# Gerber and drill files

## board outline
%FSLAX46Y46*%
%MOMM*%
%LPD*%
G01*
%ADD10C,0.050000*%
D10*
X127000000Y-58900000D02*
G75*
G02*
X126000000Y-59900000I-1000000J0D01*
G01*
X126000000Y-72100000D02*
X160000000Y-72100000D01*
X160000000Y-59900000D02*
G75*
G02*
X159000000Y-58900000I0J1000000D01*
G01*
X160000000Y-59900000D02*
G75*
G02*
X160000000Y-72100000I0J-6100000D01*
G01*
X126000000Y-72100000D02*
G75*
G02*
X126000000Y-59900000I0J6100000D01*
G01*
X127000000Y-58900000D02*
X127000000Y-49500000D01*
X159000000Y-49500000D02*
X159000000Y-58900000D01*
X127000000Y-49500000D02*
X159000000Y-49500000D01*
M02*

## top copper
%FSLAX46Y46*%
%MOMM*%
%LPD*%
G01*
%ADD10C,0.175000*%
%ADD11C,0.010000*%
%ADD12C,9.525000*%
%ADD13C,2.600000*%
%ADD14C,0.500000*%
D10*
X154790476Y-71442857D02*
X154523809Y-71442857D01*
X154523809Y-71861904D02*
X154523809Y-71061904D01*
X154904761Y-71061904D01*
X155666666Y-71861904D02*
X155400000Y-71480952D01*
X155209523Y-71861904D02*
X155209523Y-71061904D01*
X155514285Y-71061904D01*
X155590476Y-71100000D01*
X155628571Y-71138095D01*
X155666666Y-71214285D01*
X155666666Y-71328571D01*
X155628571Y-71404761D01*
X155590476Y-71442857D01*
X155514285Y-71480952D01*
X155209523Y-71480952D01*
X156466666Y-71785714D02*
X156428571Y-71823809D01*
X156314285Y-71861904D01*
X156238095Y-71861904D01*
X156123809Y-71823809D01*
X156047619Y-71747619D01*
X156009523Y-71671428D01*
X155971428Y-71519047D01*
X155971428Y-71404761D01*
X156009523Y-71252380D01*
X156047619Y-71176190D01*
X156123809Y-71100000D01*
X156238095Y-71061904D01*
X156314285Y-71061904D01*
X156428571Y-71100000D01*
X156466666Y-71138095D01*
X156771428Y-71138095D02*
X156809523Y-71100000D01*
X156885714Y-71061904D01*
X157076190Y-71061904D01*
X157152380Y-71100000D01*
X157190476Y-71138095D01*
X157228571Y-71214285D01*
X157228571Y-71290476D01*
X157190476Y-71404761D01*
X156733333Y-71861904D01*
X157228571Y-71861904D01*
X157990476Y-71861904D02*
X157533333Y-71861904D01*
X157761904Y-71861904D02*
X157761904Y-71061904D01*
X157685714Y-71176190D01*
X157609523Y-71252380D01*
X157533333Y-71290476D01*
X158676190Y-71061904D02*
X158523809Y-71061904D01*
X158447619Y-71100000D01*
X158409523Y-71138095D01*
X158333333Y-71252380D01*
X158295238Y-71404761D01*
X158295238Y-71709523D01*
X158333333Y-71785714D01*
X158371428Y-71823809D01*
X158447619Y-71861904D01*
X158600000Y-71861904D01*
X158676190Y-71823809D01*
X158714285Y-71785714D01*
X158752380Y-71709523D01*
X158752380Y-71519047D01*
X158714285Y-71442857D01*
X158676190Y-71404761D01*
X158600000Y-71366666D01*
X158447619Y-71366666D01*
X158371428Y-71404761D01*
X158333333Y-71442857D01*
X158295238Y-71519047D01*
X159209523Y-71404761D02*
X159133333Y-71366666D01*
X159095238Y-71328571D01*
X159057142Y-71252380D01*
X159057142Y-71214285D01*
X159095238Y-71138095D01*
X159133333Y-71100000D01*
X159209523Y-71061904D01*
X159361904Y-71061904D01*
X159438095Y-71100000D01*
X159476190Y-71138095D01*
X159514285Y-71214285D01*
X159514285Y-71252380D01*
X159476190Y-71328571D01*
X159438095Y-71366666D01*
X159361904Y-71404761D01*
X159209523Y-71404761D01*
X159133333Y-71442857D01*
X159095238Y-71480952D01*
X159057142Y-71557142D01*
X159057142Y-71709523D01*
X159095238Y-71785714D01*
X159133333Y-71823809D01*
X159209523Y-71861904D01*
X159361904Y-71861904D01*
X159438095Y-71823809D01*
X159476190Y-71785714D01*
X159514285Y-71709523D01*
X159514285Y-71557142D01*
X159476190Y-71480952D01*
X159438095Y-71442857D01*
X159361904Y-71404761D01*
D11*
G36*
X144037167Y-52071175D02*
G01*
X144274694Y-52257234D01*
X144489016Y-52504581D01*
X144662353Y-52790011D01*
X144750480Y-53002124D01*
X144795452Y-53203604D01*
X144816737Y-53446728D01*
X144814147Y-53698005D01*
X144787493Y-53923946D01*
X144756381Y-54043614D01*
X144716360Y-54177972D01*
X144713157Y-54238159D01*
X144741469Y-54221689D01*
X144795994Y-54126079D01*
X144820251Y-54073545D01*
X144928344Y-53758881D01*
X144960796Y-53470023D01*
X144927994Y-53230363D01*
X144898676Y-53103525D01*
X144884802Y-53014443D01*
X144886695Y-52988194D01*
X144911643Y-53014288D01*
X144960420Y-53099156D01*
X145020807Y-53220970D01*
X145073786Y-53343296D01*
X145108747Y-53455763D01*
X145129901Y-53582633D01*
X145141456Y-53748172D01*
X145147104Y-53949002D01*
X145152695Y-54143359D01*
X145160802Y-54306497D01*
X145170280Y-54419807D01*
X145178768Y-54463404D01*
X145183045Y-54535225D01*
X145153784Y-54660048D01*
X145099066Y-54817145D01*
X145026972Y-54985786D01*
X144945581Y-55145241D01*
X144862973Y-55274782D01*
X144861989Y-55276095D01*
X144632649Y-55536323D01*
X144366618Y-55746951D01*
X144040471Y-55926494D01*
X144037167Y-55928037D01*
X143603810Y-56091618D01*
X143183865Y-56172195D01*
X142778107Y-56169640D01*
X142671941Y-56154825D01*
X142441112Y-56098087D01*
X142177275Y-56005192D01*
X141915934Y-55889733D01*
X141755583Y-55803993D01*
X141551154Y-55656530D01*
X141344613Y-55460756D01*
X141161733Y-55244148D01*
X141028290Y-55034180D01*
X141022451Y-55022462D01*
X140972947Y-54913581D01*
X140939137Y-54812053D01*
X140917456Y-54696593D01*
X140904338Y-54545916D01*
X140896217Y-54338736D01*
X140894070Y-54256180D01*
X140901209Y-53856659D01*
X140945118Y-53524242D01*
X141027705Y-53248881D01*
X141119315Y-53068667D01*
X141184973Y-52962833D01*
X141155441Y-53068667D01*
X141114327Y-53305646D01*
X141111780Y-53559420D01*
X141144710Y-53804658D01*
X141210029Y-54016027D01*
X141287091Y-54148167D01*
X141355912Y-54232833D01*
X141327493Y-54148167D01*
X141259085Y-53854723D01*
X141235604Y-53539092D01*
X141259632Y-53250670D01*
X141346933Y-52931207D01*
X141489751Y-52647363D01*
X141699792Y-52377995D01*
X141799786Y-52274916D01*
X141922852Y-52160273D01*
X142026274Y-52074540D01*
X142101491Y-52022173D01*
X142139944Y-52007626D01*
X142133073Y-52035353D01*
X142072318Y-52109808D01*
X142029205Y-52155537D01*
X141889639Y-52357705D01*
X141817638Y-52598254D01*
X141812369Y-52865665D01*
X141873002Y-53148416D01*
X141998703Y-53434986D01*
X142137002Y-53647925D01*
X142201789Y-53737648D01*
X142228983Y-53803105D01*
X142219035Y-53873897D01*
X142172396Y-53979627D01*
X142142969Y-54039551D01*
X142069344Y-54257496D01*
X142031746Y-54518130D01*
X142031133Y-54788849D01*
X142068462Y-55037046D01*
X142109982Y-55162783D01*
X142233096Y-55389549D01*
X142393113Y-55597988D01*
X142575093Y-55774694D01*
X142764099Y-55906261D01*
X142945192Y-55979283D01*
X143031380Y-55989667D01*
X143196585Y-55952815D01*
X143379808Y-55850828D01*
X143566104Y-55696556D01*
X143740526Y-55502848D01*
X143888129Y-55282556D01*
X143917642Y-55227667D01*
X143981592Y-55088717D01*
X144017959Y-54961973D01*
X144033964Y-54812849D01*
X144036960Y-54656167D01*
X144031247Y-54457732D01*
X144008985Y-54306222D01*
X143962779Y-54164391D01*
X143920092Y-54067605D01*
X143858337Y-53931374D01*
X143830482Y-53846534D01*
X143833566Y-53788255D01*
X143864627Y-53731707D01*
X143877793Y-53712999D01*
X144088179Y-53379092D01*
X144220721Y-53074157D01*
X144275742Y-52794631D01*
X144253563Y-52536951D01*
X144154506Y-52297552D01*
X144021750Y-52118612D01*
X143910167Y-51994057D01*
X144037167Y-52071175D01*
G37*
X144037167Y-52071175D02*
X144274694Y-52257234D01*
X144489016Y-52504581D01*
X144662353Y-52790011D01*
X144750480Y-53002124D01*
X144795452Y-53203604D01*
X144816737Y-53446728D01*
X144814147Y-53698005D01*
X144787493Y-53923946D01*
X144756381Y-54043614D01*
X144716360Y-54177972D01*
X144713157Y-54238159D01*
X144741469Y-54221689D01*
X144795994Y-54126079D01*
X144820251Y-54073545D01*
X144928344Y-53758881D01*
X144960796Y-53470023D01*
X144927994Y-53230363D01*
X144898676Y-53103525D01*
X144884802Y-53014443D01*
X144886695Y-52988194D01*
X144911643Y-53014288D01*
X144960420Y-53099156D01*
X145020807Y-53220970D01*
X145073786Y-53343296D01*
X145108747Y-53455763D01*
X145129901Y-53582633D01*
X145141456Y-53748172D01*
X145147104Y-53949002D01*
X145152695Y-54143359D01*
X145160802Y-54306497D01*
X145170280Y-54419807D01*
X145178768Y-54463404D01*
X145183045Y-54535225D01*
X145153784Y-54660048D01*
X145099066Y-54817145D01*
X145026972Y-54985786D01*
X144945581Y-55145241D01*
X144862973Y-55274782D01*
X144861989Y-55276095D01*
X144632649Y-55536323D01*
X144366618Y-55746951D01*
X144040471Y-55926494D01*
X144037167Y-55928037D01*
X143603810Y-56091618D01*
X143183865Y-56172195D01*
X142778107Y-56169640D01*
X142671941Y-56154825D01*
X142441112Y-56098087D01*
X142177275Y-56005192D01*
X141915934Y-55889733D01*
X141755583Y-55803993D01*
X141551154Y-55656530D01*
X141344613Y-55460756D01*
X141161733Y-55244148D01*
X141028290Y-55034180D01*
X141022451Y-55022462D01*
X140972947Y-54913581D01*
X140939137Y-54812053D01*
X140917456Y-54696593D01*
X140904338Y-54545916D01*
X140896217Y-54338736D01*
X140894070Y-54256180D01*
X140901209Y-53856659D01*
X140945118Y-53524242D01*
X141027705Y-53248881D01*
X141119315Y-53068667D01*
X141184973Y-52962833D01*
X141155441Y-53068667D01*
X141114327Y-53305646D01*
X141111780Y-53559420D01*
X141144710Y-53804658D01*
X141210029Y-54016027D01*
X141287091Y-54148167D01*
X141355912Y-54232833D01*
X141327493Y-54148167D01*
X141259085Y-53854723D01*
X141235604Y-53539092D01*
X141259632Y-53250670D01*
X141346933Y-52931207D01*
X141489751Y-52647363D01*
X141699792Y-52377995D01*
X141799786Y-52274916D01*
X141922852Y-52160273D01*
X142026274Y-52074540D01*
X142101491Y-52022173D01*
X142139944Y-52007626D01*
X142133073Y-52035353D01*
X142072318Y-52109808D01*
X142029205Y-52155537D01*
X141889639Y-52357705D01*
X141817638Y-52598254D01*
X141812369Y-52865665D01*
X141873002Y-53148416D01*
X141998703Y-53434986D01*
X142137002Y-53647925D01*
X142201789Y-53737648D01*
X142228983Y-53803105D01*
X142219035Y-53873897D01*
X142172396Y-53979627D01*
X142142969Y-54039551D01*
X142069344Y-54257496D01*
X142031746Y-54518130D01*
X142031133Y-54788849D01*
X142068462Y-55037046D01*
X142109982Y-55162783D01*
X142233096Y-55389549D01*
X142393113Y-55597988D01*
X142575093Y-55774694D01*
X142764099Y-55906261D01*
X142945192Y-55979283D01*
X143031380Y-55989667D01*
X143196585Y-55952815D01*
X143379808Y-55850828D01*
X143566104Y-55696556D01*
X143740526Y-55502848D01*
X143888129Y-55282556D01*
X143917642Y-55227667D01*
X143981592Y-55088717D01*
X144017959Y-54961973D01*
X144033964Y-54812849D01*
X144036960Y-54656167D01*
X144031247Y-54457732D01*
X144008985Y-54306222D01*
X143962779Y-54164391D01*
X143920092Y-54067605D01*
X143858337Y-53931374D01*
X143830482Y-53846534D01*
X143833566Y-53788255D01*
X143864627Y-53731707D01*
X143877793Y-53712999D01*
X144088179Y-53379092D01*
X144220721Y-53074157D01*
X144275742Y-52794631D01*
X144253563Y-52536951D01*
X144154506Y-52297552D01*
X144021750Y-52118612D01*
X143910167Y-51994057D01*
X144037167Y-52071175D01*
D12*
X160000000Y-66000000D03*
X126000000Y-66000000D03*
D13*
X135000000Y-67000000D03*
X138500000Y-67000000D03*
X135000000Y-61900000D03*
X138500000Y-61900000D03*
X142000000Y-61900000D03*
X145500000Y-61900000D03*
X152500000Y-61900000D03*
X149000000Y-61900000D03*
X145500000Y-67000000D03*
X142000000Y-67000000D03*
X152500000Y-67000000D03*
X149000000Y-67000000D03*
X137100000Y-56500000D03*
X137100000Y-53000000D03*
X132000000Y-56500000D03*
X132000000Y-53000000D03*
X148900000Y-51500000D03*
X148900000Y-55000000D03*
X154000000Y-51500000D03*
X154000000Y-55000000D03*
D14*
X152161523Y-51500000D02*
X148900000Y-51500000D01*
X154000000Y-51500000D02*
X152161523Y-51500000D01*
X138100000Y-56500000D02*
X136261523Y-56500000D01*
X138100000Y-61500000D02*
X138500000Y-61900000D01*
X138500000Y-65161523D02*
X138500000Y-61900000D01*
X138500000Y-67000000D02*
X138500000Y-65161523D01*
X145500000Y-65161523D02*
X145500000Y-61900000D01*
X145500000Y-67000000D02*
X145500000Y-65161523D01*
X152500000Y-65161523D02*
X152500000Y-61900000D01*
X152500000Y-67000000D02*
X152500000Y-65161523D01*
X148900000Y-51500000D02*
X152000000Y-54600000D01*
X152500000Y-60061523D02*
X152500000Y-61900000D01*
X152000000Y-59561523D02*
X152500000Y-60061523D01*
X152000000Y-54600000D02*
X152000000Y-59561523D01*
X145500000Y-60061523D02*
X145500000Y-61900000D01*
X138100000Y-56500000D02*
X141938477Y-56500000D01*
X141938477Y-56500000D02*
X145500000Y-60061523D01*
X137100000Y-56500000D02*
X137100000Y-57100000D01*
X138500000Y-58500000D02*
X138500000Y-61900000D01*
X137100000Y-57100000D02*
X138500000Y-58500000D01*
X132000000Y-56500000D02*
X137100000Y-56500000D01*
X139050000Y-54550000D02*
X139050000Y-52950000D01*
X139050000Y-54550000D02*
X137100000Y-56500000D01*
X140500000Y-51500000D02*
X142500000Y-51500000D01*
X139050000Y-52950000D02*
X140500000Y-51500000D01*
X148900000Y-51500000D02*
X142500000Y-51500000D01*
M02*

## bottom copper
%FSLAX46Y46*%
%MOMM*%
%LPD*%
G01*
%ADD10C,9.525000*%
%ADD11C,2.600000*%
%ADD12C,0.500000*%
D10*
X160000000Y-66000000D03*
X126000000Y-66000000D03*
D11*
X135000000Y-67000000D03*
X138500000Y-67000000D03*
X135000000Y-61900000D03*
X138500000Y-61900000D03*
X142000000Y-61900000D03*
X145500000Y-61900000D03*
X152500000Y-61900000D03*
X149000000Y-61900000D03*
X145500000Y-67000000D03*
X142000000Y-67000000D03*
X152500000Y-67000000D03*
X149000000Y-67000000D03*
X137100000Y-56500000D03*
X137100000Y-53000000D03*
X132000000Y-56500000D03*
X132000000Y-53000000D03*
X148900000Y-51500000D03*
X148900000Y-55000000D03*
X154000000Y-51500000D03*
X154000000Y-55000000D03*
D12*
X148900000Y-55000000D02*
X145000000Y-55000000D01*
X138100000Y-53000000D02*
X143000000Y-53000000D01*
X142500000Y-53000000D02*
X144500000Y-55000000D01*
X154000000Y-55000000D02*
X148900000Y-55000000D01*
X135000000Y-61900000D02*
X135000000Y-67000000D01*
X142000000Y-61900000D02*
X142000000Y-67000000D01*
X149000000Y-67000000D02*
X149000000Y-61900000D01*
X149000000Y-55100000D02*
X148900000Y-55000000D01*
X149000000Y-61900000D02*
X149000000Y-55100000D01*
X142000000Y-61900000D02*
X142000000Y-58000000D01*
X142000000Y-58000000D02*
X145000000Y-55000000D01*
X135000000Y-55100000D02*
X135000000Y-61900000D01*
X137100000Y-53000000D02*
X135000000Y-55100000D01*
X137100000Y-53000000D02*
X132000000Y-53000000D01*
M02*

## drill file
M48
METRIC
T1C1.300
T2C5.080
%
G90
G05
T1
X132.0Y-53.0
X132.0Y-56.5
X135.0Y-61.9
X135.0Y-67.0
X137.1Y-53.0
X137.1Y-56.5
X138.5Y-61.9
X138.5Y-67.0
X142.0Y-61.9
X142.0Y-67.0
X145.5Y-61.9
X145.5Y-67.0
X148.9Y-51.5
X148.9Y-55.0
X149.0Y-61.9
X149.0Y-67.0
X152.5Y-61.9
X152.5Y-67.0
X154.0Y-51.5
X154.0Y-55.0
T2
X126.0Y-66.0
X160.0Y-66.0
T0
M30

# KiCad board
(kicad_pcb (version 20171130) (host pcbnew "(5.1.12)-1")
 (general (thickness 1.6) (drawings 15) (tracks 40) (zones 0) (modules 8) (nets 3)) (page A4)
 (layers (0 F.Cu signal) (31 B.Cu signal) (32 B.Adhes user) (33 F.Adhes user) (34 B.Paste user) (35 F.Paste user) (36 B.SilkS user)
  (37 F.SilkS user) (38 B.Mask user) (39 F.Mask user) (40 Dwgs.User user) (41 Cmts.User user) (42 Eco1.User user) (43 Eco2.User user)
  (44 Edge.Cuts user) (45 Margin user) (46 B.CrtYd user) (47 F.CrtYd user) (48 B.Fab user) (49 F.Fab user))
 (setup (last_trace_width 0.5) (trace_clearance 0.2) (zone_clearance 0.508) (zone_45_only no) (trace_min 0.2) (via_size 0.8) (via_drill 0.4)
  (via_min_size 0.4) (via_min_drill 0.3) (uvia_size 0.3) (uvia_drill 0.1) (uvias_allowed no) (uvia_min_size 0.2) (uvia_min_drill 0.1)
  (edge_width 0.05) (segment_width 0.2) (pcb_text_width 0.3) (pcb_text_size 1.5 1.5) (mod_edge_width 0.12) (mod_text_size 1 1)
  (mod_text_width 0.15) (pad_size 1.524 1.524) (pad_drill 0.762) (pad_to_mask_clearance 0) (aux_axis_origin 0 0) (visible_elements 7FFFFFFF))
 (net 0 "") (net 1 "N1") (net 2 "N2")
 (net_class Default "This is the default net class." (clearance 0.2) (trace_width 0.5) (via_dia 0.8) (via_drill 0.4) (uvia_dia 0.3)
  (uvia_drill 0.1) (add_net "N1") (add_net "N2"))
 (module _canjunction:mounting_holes (layer F.Cu) (at 126 66)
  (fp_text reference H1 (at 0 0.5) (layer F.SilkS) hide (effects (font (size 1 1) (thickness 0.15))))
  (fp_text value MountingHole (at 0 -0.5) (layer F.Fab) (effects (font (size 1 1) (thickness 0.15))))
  (pad "" thru_hole circle (at 34 0) (size 9.525 9.525) (drill 5.08) (layers *.Cu *.Mask))
  (pad "" thru_hole circle (at 0 0) (size 9.525 9.525) (drill 5.08) (layers *.Cu *.Mask)))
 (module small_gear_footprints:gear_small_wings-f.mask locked (layer F.Cu) (at 143 54)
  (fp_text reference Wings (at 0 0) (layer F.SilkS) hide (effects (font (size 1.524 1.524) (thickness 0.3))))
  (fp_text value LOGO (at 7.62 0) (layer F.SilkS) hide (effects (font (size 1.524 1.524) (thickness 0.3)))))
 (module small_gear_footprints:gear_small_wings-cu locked (layer F.Cu) (at 143 54)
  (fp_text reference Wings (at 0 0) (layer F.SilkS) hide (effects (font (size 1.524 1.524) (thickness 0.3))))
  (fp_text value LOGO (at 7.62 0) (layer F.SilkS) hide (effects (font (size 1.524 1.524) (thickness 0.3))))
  (fp_poly
   (pts (xy 1.037167 -1.928825) (xy 1.274694 -1.742766) (xy 1.489016 -1.495419) (xy 1.662353 -1.209989) (xy 1.75048 -0.997876)
    (xy 1.795452 -0.796396) (xy 1.816737 -0.553272) (xy 1.814147 -0.301995) (xy 1.787493 -0.076054) (xy 1.756381 0.043614)
    (xy 1.71636 0.177972) (xy 1.713157 0.238159) (xy 1.741469 0.221689) (xy 1.795994 0.126079) (xy 1.820251 0.073545)
    (xy 1.928344 -0.241119) (xy 1.960796 -0.529977) (xy 1.927994 -0.769637) (xy 1.898676 -0.896475) (xy 1.884802 -0.985557)
    (xy 1.886695 -1.011806) (xy 1.911643 -0.985712) (xy 1.96042 -0.900844) (xy 2.020807 -0.77903) (xy 2.073786 -0.656704)
    (xy 2.108747 -0.544237) (xy 2.129901 -0.417367) (xy 2.141456 -0.251828) (xy 2.147104 -0.050998) (xy 2.152695 0.143359)
    (xy 2.160802 0.306497) (xy 2.17028 0.419807) (xy 2.178768 0.463404) (xy 2.183045 0.535225) (xy 2.153784 0.660048) (xy 2.099066 0.817145)
    (xy 2.026972 0.985786) (xy 1.945581 1.145241) (xy 1.862973 1.274782) (xy 1.861989 1.276095) (xy 1.632649 1.536323)
    (xy 1.366618 1.746951) (xy 1.040471 1.926494) (xy 1.037167 1.928037) (xy 0.60381 2.091618) (xy 0.183865 2.172195) (xy -0.221893 2.16964)
    (xy -0.328059 2.154825) (xy -0.558888 2.098087) (xy -0.822725 2.005192) (xy -1.084066 1.889733) (xy -1.244417 1.803993)
    (xy -1.448846 1.65653) (xy -1.655387 1.460756) (xy -1.838267 1.244148) (xy -1.97171 1.03418) (xy -1.977549 1.022462)
    (xy -2.027053 0.913581) (xy -2.060863 0.812053) (xy -2.082544 0.696593) (xy -2.095662 0.545916) (xy -2.103783 0.338736)
    (xy -2.10593 0.25618) (xy -2.098791 -0.143341) (xy -2.054882 -0.475758) (xy -1.972295 -0.751119) (xy -1.880685 -0.931333)
    (xy -1.815027 -1.037167) (xy -1.844559 -0.931333) (xy -1.885673 -0.694354) (xy -1.88822 -0.44058) (xy -1.85529 -0.195342)
    (xy -1.789971 0.016027) (xy -1.712909 0.148167) (xy -1.644088 0.232833) (xy -1.672507 0.148167) (xy -1.740915 -0.145277)
    (xy -1.764396 -0.460908) (xy -1.740368 -0.74933) (xy -1.653067 -1.068793) (xy -1.510249 -1.352637) (xy -1.300208 -1.622005)
    (xy -1.200214 -1.725084) (xy -1.077148 -1.839727) (xy -0.973726 -1.92546) (xy -0.898509 -1.977827) (xy -0.860056 -1.992374)
    (xy -0.866927 -1.964647) (xy -0.927682 -1.890192) (xy -0.970795 -1.844463) (xy -1.110361 -1.642295) (xy -1.182362 -1.401746)
    (xy -1.187631 -1.134335) (xy -1.126998 -0.851584) (xy -1.001297 -0.565014) (xy -0.862998 -0.352075) (xy -0.798211 -0.262352)
    (xy -0.771017 -0.196895) (xy -0.780965 -0.126103) (xy -0.827604 -0.020373) (xy -0.857031 0.039551) (xy -0.930656 0.257496)
    (xy -0.968254 0.51813) (xy -0.968867 0.788849) (xy -0.931538 1.037046) (xy -0.890018 1.162783) (xy -0.766904 1.389549)
    (xy -0.606887 1.597988) (xy -0.424907 1.774694) (xy -0.235901 1.906261) (xy -0.054808 1.979283) (xy 0.03138 1.989667)
    (xy 0.196585 1.952815) (xy 0.379808 1.850828) (xy 0.566104 1.696556) (xy 0.740526 1.502848) (xy 0.888129 1.282556)
    (xy 0.917642 1.227667) (xy 0.981592 1.088717) (xy 1.017959 0.961973) (xy 1.033964 0.812849) (xy 1.03696 0.656167) (xy 1.031247 0.457732)
    (xy 1.008985 0.306222) (xy 0.962779 0.164391) (xy 0.920092 0.067605) (xy 0.858337 -0.068626) (xy 0.830482 -0.153466)
    (xy 0.833566 -0.211745) (xy 0.864627 -0.268293) (xy 0.877793 -0.287001) (xy 1.088179 -0.620908) (xy 1.220721 -0.925843)
    (xy 1.275742 -1.205369) (xy 1.253563 -1.463049) (xy 1.154506 -1.702448) (xy 1.02175 -1.881388) (xy 0.910167 -2.005943)
    (xy 1.037167 -1.928825))
   (layer F.Cu) (width 0.01)))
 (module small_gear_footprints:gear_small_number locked (layer F.Cu) (at 143 54)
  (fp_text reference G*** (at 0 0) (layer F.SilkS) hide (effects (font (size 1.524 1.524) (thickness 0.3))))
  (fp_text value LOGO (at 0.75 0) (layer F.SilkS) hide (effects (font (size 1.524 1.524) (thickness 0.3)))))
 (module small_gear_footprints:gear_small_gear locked (layer F.Cu) (at 143 54)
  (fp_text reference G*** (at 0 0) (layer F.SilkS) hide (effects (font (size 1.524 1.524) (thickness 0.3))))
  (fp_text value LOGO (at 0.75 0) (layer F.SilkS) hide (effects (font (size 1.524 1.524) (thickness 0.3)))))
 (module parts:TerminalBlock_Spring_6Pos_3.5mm (layer F.Cu) (at 135 67)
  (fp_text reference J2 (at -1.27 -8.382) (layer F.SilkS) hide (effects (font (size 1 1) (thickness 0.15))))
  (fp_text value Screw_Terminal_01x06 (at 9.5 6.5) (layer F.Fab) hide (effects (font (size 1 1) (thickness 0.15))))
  (pad 1 thru_hole circle (at 0 0) (size 2.6 2.6) (drill 1.3) (layers *.Cu *.Mask) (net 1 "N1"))
  (pad 2 thru_hole circle (at 3.5 0) (size 2.6 2.6) (drill 1.3) (layers *.Cu *.Mask) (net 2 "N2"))
  (pad 1 thru_hole circle (at 0 -5.1) (size 2.6 2.6) (drill 1.3) (layers *.Cu *.Mask) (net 1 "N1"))
  (pad 2 thru_hole circle (at 3.5 -5.1) (size 2.6 2.6) (drill 1.3) (layers *.Cu *.Mask) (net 2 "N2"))
  (pad 3 thru_hole circle (at 7 -5.1) (size 2.6 2.6) (drill 1.3) (layers *.Cu *.Mask) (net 1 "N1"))
  (pad 4 thru_hole circle (at 10.5 -5.1) (size 2.6 2.6) (drill 1.3) (layers *.Cu *.Mask) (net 2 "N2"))
  (pad 6 thru_hole circle (at 17.5 -5.1) (size 2.6 2.6) (drill 1.3) (layers *.Cu *.Mask) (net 2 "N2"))
  (pad 5 thru_hole circle (at 14 -5.1) (size 2.6 2.6) (drill 1.3) (layers *.Cu *.Mask) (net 1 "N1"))
  (pad 4 thru_hole circle (at 10.5 0) (size 2.6 2.6) (drill 1.3) (layers *.Cu *.Mask) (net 2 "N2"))
  (pad 3 thru_hole circle (at 7 0) (size 2.6 2.6) (drill 1.3) (layers *.Cu *.Mask) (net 1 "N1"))
  (pad 6 thru_hole circle (at 17.5 0) (size 2.6 2.6) (drill 1.3) (layers *.Cu *.Mask) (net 2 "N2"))
  (pad 5 thru_hole circle (at 14 0) (size 2.6 2.6) (drill 1.3) (layers *.Cu *.Mask) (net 1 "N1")))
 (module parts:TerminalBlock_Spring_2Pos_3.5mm (layer F.Cu) (at 132 53 270)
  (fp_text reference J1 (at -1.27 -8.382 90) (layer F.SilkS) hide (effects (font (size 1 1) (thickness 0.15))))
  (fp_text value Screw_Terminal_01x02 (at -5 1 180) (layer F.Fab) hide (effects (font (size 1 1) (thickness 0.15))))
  (pad 2 thru_hole circle (at 3.5 -5.1 270) (size 2.6 2.6) (drill 1.3) (layers *.Cu *.Mask) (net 2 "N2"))
  (pad 1 thru_hole circle (at 0 -5.1 270) (size 2.6 2.6) (drill 1.3) (layers *.Cu *.Mask) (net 1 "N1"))
  (pad 2 thru_hole circle (at 3.5 0 270) (size 2.6 2.6) (drill 1.3) (layers *.Cu *.Mask) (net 2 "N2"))
  (pad 1 thru_hole circle (at 0 0 270) (size 2.6 2.6) (drill 1.3) (layers *.Cu *.Mask) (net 1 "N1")))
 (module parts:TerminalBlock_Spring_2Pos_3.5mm (layer F.Cu) (at 154 55 90)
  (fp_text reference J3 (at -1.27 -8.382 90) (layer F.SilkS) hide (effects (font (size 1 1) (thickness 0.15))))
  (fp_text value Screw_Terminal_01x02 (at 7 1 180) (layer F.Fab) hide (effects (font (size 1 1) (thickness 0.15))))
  (pad 2 thru_hole circle (at 3.5 -5.1 90) (size 2.6 2.6) (drill 1.3) (layers *.Cu *.Mask) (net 2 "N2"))
  (pad 1 thru_hole circle (at 0 -5.1 90) (size 2.6 2.6) (drill 1.3) (layers *.Cu *.Mask) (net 1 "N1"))
  (pad 2 thru_hole circle (at 3.5 0 90) (size 2.6 2.6) (drill 1.3) (layers *.Cu *.Mask) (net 2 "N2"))
  (pad 1 thru_hole circle (at 0 0 90) (size 2.6 2.6) (drill 1.3) (layers *.Cu *.Mask) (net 1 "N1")))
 (gr_arc (start 126 58.9) (end 126 59.9) (angle -90) (layer Edge.Cuts) (width 0.05))
 (gr_line (start 126 72.1) (end 160 72.1) (layer Edge.Cuts) (width 0.05))
 (gr_arc (start 160 58.9) (end 159 58.9) (angle -90) (layer Edge.Cuts) (width 0.05))
 (gr_arc (start 160 66) (end 160 72.1) (angle -180) (layer Edge.Cuts) (width 0.05))
 (gr_arc (start 126 66) (end 126 59.9) (angle -180) (layer Edge.Cuts) (width 0.05))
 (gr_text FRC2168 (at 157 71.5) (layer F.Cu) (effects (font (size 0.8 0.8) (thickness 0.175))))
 (gr_line (start 127 58.9) (end 127 49.5) (layer Edge.Cuts) (width 0.05))
 (gr_line (start 159 49.5) (end 159 58.9) (layer Edge.Cuts) (width 0.05))
 (gr_line (start 127 49.5) (end 159 49.5) (layer Edge.Cuts) (width 0.05))
 (segment (start 148.9 55) (end 145 55) (width 0.5) (layer B.Cu) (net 1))
 (segment (start 138.1 53) (end 143 53) (width 0.5) (layer B.Cu) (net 1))
 (segment (start 142.5 53) (end 144.5 55) (width 0.5) (layer B.Cu) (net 1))
 (segment (start 154 55) (end 148.9 55) (width 0.5) (layer B.Cu) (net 1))
 (segment (start 135 61.9) (end 135 67) (width 0.5) (layer B.Cu) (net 1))
 (segment (start 142 61.9) (end 142 67) (width 0.5) (layer B.Cu) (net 1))
 (segment (start 149 67) (end 149 61.9) (width 0.5) (layer B.Cu) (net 1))
 (segment (start 149 55.1) (end 148.9 55) (width 0.5) (layer B.Cu) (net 1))
 (segment (start 149 61.9) (end 149 55.1) (width 0.5) (layer B.Cu) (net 1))
 (segment (start 142 61.9) (end 142 58) (width 0.5) (layer B.Cu) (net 1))
 (segment (start 142 58) (end 145 55) (width 0.5) (layer B.Cu) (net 1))
 (segment (start 135 55.1) (end 135 61.9) (width 0.5) (layer B.Cu) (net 1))
 (segment (start 137.1 53) (end 135 55.1) (width 0.5) (layer B.Cu) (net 1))
 (segment (start 137.1 53) (end 132 53) (width 0.5) (layer B.Cu) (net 1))
 (segment (start 152.161523 51.5) (end 148.9 51.5) (width 0.5) (layer F.Cu) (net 2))
 (segment (start 154 51.5) (end 152.161523 51.5) (width 0.5) (layer F.Cu) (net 2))
 (segment (start 138.1 56.5) (end 136.261523 56.5) (width 0.5) (layer F.Cu) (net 2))
 (segment (start 138.1 61.5) (end 138.5 61.9) (width 0.5) (layer F.Cu) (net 2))
 (segment (start 138.5 65.161523) (end 138.5 61.9) (width 0.5) (layer F.Cu) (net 2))
 (segment (start 138.5 67) (end 138.5 65.161523) (width 0.5) (layer F.Cu) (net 2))
 (segment (start 145.5 65.161523) (end 145.5 61.9) (width 0.5) (layer F.Cu) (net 2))
 (segment (start 145.5 67) (end 145.5 65.161523) (width 0.5) (layer F.Cu) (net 2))
 (segment (start 152.5 65.161523) (end 152.5 61.9) (width 0.5) (layer F.Cu) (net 2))
 (segment (start 152.5 67) (end 152.5 65.161523) (width 0.5) (layer F.Cu) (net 2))
 (segment (start 148.9 51.5) (end 152 54.6) (width 0.5) (layer F.Cu) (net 2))
 (segment (start 152.5 60.061523) (end 152.5 61.9) (width 0.5) (layer F.Cu) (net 2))
 (segment (start 152 59.561523) (end 152.5 60.061523) (width 0.5) (layer F.Cu) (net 2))
 (segment (start 152 54.6) (end 152 59.561523) (width 0.5) (layer F.Cu) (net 2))
 (segment (start 145.5 60.061523) (end 145.5 61.9) (width 0.5) (layer F.Cu) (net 2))
 (segment (start 138.1 56.5) (end 141.938477 56.5) (width 0.5) (layer F.Cu) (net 2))
 (segment (start 141.938477 56.5) (end 145.5 60.061523) (width 0.5) (layer F.Cu) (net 2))
 (segment (start 137.1 56.5) (end 137.1 57.1) (width 0.5) (layer F.Cu) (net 2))
 (segment (start 138.5 58.5) (end 138.5 61.9) (width 0.5) (layer F.Cu) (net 2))
 (segment (start 137.1 57.1) (end 138.5 58.5) (width 0.5) (layer F.Cu) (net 2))
 (segment (start 132 56.5) (end 137.1 56.5) (width 0.5) (layer F.Cu) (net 2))
 (segment (start 139.05 54.55) (end 139.05 52.95) (width 0.5) (layer F.Cu) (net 2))
 (segment (start 139.05 54.55) (end 137.1 56.5) (width 0.5) (layer F.Cu) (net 2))
 (segment (start 140.5 51.5) (end 142.5 51.5) (width 0.5) (layer F.Cu) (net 2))
 (segment (start 139.05 52.95) (end 140.5 51.5) (width 0.5) (layer F.Cu) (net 2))
 (segment (start 148.9 51.5) (end 142.5 51.5) (width 0.5) (layer F.Cu) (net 2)))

